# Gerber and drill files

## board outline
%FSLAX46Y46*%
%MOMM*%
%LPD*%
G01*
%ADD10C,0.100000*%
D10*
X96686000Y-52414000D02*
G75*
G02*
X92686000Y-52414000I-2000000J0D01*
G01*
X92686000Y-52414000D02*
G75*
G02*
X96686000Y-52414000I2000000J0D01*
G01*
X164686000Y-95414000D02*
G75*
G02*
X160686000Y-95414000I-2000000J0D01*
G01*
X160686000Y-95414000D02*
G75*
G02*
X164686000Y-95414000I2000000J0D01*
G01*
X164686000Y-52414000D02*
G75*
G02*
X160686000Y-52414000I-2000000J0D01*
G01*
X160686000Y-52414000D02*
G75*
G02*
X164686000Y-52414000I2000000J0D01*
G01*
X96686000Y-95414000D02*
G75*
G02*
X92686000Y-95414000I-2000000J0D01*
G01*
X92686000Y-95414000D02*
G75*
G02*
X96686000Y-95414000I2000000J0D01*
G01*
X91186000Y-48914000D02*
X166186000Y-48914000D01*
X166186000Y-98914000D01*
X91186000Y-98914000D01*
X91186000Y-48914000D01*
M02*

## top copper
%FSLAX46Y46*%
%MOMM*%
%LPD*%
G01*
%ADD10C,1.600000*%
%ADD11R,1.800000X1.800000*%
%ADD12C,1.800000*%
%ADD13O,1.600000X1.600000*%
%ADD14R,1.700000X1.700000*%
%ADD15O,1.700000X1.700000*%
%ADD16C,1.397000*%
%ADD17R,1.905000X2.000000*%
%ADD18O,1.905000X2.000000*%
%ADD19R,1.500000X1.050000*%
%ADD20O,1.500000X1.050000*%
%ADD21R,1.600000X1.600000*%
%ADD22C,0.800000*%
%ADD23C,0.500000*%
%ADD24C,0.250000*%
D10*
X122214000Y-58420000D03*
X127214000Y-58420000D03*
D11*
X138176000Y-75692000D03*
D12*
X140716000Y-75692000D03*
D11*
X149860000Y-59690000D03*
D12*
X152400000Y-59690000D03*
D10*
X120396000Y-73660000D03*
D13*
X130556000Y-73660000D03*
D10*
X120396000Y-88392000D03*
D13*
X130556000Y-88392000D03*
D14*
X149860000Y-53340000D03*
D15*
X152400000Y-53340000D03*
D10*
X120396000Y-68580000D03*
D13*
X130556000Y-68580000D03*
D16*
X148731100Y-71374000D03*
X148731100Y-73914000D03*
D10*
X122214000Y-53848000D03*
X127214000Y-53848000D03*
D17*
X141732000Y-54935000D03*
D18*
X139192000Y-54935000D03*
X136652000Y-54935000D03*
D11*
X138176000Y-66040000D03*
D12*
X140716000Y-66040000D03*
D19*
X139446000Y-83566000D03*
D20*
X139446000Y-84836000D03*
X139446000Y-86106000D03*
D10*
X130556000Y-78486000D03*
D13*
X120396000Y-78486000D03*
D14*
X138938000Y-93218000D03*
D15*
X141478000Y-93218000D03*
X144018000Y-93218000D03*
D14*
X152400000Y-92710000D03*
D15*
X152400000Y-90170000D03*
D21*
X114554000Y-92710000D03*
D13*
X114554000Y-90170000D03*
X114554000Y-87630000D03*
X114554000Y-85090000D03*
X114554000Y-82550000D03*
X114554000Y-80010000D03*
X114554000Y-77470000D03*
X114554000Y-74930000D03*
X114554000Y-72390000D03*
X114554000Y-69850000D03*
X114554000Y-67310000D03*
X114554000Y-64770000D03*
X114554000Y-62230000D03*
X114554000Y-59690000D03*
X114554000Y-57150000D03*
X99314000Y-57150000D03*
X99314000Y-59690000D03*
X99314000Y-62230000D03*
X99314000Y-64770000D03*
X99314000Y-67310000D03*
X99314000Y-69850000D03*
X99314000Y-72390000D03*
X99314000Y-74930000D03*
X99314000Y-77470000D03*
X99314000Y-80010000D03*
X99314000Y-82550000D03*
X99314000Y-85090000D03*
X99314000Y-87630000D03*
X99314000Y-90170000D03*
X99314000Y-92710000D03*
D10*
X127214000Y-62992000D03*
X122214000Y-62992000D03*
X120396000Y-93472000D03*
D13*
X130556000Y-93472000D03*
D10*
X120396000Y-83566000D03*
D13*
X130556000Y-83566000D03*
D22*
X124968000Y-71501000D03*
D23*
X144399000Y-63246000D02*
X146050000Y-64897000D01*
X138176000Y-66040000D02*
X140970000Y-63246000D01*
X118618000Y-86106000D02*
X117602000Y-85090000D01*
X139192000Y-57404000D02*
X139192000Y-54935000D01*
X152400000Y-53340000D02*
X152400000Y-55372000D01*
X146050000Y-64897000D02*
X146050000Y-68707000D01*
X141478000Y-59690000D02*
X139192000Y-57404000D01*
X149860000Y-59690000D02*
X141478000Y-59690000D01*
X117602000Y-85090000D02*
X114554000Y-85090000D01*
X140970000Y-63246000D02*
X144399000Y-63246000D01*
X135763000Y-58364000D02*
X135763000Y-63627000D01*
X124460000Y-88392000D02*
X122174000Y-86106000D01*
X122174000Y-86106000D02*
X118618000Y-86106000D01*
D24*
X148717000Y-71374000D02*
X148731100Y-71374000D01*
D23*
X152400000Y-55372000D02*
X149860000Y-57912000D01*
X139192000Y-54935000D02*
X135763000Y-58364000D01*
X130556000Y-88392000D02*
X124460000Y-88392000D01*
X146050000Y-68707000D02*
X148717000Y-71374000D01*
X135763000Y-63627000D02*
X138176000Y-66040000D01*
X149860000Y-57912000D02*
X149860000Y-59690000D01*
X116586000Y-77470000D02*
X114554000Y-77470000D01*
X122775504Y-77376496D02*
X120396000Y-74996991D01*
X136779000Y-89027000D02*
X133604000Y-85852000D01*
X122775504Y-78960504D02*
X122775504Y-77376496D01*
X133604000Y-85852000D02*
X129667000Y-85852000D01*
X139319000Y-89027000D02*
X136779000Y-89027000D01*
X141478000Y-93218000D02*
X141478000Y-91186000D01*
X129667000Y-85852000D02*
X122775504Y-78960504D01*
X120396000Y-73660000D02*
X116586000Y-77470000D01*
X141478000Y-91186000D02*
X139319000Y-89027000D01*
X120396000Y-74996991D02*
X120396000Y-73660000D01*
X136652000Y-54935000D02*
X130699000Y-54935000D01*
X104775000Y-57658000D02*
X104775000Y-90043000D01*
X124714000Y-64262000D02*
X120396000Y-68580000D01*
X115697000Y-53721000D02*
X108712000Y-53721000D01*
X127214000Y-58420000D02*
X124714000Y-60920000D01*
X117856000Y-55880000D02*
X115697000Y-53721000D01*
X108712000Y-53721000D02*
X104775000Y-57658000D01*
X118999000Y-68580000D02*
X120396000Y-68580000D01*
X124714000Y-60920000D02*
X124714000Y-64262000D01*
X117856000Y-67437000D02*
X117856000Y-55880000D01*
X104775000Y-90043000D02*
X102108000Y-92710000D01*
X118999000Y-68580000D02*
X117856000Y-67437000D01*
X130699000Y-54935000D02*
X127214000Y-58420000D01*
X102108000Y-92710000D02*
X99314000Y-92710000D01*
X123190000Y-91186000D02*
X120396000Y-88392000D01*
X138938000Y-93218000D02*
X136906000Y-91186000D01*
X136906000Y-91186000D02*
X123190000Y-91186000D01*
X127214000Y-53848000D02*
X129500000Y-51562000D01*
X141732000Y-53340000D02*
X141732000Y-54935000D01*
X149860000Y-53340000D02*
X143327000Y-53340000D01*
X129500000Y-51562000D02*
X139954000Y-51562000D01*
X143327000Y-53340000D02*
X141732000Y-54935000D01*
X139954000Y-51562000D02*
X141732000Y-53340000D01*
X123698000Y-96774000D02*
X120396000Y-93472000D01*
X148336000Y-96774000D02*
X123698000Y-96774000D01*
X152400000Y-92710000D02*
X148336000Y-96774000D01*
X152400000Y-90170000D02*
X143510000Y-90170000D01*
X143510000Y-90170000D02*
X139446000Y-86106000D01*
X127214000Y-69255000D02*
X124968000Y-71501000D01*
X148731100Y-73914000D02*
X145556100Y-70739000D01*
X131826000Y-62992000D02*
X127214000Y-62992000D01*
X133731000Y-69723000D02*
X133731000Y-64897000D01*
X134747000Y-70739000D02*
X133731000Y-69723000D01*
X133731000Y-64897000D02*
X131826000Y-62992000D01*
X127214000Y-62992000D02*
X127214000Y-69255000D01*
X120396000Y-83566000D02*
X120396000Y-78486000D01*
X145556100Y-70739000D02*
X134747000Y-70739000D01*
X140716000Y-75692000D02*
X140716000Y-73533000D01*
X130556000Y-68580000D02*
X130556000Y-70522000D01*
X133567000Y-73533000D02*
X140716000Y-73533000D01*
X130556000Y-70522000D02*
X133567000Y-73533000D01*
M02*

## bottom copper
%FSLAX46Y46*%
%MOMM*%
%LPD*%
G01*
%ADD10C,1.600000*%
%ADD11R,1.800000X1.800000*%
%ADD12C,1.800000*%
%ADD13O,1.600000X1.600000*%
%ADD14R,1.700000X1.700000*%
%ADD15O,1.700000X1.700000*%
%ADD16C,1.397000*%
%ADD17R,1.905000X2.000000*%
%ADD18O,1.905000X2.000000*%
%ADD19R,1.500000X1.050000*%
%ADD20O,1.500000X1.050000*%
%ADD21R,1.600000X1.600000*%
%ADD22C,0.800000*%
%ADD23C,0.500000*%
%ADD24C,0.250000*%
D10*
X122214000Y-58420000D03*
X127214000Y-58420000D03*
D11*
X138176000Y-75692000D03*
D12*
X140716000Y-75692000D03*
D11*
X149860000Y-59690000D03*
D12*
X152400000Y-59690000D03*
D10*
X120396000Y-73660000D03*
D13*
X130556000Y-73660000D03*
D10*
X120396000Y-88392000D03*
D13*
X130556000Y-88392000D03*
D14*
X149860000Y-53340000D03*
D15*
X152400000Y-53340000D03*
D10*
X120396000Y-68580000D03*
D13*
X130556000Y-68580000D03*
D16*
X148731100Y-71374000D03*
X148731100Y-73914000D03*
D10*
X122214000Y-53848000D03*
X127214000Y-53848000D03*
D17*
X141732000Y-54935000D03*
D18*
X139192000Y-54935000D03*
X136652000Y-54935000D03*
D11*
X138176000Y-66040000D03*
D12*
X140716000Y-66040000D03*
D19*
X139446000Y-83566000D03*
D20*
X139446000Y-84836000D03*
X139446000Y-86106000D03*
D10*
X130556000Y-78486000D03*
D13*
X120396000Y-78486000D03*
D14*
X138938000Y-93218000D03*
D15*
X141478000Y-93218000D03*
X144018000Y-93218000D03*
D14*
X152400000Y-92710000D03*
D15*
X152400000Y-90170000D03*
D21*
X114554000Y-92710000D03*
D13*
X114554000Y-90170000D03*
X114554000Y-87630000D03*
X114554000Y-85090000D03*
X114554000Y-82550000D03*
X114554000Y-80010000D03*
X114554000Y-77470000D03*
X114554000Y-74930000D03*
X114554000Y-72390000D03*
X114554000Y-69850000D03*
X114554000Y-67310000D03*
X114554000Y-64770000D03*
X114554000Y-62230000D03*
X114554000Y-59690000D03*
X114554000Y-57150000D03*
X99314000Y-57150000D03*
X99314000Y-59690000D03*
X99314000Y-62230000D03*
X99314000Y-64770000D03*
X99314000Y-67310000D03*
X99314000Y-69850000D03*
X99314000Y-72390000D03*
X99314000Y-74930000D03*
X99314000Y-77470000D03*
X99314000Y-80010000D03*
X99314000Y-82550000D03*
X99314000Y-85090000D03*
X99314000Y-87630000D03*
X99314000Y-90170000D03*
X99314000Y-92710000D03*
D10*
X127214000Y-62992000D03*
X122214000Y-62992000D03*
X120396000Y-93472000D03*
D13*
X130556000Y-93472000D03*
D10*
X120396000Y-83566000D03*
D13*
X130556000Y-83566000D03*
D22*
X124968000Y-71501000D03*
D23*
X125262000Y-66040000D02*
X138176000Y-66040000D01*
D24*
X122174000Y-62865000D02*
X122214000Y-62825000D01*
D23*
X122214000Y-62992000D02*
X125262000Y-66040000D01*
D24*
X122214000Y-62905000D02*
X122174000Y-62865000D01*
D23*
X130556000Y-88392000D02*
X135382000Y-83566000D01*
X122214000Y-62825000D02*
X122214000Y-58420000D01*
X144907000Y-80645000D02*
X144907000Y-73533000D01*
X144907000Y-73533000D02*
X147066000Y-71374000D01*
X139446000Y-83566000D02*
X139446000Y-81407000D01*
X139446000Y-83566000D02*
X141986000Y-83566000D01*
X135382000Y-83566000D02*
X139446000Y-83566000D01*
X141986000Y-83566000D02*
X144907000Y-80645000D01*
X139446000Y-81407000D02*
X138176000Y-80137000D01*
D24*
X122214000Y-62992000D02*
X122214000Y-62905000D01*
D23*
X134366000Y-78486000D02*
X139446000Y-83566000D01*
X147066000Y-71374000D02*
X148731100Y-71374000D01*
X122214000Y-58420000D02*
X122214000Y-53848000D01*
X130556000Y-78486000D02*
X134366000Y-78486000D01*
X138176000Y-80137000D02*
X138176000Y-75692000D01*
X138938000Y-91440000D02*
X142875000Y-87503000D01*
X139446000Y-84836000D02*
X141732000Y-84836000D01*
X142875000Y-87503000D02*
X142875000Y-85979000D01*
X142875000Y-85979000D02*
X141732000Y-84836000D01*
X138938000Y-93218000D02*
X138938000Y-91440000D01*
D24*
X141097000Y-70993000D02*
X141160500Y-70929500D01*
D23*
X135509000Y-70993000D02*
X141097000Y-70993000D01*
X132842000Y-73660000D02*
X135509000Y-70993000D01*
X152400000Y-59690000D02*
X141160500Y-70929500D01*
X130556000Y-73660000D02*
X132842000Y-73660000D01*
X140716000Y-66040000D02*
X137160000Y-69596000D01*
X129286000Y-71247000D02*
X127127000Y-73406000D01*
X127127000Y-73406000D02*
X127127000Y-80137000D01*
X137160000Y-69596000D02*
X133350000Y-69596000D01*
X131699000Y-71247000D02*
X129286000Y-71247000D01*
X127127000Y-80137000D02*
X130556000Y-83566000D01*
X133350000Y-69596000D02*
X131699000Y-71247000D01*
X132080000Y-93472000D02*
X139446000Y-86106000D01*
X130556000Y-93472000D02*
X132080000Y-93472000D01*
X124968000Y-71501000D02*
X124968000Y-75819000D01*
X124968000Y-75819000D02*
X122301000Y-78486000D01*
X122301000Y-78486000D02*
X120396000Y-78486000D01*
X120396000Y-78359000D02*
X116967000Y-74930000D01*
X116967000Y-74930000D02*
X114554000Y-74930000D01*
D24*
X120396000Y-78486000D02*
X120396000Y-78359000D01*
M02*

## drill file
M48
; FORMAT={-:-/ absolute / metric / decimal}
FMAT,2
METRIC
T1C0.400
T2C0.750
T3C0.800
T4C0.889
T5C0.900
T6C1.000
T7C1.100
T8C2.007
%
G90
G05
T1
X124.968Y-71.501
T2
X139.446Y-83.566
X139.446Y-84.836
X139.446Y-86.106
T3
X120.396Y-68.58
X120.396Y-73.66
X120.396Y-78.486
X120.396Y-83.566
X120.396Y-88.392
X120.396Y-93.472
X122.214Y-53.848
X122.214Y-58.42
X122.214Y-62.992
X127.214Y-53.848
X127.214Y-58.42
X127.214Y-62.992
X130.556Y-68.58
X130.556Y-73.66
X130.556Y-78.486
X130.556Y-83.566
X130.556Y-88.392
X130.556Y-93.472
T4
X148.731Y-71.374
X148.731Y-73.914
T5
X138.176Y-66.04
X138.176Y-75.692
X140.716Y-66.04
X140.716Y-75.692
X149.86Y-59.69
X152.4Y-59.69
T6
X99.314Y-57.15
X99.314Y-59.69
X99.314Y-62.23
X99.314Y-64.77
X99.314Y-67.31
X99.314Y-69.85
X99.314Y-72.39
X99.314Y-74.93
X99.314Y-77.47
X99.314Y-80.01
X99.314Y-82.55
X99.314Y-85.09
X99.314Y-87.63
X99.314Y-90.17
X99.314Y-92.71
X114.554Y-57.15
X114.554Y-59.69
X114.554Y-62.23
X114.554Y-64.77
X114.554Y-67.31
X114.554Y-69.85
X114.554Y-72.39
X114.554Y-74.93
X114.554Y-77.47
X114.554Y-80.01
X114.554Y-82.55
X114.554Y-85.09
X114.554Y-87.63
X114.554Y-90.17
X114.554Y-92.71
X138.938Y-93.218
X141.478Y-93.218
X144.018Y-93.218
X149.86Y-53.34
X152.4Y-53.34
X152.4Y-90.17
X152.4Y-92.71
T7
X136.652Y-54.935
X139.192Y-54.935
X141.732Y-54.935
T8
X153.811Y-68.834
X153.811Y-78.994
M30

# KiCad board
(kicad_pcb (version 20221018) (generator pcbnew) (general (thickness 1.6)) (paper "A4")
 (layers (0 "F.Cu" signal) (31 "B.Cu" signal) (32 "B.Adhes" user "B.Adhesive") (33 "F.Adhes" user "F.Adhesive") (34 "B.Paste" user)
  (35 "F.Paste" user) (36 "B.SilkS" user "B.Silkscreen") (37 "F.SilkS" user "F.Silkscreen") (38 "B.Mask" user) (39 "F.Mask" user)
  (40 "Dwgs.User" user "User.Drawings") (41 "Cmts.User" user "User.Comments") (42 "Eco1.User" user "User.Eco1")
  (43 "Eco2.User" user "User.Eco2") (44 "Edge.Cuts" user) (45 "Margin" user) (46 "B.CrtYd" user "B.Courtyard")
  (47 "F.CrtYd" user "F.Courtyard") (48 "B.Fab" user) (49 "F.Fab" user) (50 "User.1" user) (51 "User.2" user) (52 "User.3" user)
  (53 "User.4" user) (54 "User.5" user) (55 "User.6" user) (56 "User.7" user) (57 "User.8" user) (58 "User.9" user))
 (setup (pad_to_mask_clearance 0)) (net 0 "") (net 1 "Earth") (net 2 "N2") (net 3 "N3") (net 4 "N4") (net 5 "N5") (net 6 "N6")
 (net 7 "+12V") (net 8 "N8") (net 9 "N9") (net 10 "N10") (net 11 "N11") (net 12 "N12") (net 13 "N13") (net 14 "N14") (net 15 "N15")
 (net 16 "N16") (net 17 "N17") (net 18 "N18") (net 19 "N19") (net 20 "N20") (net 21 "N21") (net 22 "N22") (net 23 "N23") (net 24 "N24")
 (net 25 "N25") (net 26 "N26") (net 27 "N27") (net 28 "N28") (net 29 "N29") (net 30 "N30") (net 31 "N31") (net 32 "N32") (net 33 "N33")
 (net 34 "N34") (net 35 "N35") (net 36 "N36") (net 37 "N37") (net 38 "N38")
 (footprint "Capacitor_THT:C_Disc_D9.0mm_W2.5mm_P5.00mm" (layer "F.Cu") (at 122.214 58.42)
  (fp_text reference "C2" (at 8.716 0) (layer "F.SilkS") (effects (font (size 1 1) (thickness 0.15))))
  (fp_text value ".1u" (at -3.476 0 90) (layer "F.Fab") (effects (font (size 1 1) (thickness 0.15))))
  (pad "1" thru_hole circle (at 0 0) (size 1.6 1.6) (drill 0.8) (layers "*.Cu" "*.Mask") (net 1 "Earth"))
  (pad "2" thru_hole circle (at 5 0) (size 1.6 1.6) (drill 0.8) (layers "*.Cu" "*.Mask") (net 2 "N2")))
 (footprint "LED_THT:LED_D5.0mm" (layer "F.Cu") (at 138.176 75.692)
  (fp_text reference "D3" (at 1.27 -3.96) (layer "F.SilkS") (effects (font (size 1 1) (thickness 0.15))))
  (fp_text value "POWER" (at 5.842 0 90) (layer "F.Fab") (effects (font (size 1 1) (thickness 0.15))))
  (pad "1" thru_hole rect (at 0 0) (size 1.8 1.8) (drill 0.9) (layers "*.Cu" "*.Mask") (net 1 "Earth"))
  (pad "2" thru_hole circle (at 2.54 0) (size 1.8 1.8) (drill 0.9) (layers "*.Cu" "*.Mask") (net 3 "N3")))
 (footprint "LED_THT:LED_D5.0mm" (layer "F.Cu") (at 149.86 59.69)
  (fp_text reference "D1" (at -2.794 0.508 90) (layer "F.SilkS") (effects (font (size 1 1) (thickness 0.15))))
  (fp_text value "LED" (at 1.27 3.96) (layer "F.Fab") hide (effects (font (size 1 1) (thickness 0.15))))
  (pad "1" thru_hole rect (at 0 0) (size 1.8 1.8) (drill 0.9) (layers "*.Cu" "*.Mask") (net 1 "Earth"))
  (pad "2" thru_hole circle (at 2.54 0) (size 1.8 1.8) (drill 0.9) (layers "*.Cu" "*.Mask") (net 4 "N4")))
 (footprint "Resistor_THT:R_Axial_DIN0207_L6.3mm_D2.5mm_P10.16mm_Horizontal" (layer "F.Cu") (at 120.396 73.66)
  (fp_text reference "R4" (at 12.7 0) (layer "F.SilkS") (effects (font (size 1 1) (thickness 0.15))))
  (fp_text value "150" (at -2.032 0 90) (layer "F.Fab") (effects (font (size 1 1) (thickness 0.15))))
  (pad "1" thru_hole circle (at 0 0) (size 1.6 1.6) (drill 0.8) (layers "*.Cu" "*.Mask") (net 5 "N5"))
  (pad "2" thru_hole oval (at 10.16 0) (size 1.6 1.6) (drill 0.8) (layers "*.Cu" "*.Mask") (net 4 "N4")))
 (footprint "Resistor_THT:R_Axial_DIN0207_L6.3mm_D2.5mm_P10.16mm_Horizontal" (layer "F.Cu") (at 120.396 88.392)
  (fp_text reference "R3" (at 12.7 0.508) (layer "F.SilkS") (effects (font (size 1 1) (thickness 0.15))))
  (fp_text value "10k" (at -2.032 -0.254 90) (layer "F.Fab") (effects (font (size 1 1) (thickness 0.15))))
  (pad "1" thru_hole circle (at 0 0) (size 1.6 1.6) (drill 0.8) (layers "*.Cu" "*.Mask") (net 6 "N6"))
  (pad "2" thru_hole oval (at 10.16 0) (size 1.6 1.6) (drill 0.8) (layers "*.Cu" "*.Mask") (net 1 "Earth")))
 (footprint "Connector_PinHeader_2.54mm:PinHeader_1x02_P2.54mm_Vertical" (layer "F.Cu") (at 149.86 53.34 90)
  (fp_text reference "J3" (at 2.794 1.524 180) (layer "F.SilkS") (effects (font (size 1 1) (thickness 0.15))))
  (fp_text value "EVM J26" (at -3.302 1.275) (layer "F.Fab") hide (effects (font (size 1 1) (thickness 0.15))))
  (pad "1" thru_hole rect (at 0 0 90) (size 1.7 1.7) (drill 1) (layers "*.Cu" "*.Mask") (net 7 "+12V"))
  (pad "2" thru_hole oval (at 0 2.54 90) (size 1.7 1.7) (drill 1) (layers "*.Cu" "*.Mask") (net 1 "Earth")))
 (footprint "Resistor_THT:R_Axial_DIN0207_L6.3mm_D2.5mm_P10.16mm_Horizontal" (layer "F.Cu") (at 120.396 68.58)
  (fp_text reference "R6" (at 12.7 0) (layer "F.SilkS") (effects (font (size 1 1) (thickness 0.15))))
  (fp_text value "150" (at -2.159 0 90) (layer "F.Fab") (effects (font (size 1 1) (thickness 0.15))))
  (pad "1" thru_hole circle (at 0 0) (size 1.6 1.6) (drill 0.8) (layers "*.Cu" "*.Mask") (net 2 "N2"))
  (pad "2" thru_hole oval (at 10.16 0) (size 1.6 1.6) (drill 0.8) (layers "*.Cu" "*.Mask") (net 3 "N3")))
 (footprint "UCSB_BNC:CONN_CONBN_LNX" (layer "F.Cu") (at 156.186 73.914 -90)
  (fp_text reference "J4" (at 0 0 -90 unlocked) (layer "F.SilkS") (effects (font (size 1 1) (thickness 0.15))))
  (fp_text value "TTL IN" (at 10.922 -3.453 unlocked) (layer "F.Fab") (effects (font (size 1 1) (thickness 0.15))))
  (pad "" np_thru_hole circle (at -5.08 2.3749 270) (size 2.0066 2.0066) (drill 2.0066) (layers "*.Cu" "*.Mask"))
  (pad "" np_thru_hole circle (at 5.08 2.3749 270) (size 2.0066 2.0066) (drill 2.0066) (layers "*.Cu" "*.Mask"))
  (pad "1" thru_hole circle (at -2.54 7.4549 270) (size 1.397 1.397) (drill 0.889) (layers "*.Cu" "*.Mask") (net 1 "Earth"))
  (pad "2" thru_hole circle (at 0 7.4549 270) (size 1.397 1.397) (drill 0.889) (layers "*.Cu" "*.Mask") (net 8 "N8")))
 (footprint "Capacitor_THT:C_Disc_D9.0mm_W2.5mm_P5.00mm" (layer "F.Cu") (at 122.214 53.848)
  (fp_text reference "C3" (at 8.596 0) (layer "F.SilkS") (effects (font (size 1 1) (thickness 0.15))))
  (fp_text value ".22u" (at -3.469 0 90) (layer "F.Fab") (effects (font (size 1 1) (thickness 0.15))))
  (pad "1" thru_hole circle (at 0 0) (size 1.6 1.6) (drill 0.8) (layers "*.Cu" "*.Mask") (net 1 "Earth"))
  (pad "2" thru_hole circle (at 5 0) (size 1.6 1.6) (drill 0.8) (layers "*.Cu" "*.Mask") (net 7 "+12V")))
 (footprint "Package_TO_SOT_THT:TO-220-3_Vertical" (layer "F.Cu") (at 141.732 54.935 180)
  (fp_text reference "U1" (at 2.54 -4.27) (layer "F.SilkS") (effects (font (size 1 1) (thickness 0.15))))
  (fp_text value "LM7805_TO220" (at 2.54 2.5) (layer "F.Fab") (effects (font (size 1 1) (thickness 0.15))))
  (pad "1" thru_hole rect (at 0 0 180) (size 1.905 2) (drill 1.1) (layers "*.Cu" "*.Mask") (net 7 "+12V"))
  (pad "2" thru_hole oval (at 2.54 0 180) (size 1.905 2) (drill 1.1) (layers "*.Cu" "*.Mask") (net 1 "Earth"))
  (pad "3" thru_hole oval (at 5.08 0 180) (size 1.905 2) (drill 1.1) (layers "*.Cu" "*.Mask") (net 2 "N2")))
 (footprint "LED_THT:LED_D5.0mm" (layer "F.Cu") (at 138.176 66.04)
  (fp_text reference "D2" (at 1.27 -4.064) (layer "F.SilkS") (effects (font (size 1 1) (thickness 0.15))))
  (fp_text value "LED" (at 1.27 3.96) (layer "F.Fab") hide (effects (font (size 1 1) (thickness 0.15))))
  (pad "1" thru_hole rect (at 0 0) (size 1.8 1.8) (drill 0.9) (layers "*.Cu" "*.Mask") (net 1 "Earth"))
  (pad "2" thru_hole circle (at 2.54 0) (size 1.8 1.8) (drill 0.9) (layers "*.Cu" "*.Mask") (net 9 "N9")))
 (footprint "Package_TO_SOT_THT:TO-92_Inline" (layer "F.Cu") (at 139.446 83.566 -90)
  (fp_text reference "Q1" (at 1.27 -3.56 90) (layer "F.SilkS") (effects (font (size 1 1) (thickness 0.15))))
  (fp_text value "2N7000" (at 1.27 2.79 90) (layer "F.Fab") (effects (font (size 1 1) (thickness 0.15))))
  (pad "1" thru_hole rect (at 0 0 270) (size 1.05 1.5) (drill 0.75) (layers "*.Cu" "*.Mask") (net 1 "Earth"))
  (pad "2" thru_hole oval (at 1.27 0 270) (size 1.05 1.5) (drill 0.75) (layers "*.Cu" "*.Mask") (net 6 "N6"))
  (pad "3" thru_hole oval (at 2.54 0 270) (size 1.05 1.5) (drill 0.75) (layers "*.Cu" "*.Mask") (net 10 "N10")))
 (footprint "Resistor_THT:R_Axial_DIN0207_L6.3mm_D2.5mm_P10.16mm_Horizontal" (layer "F.Cu") (at 130.556 78.486 180)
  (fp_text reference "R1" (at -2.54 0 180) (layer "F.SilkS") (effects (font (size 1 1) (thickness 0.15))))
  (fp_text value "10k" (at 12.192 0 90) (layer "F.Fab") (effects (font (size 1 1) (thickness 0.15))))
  (pad "1" thru_hole circle (at 0 0 180) (size 1.6 1.6) (drill 0.8) (layers "*.Cu" "*.Mask") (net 1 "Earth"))
  (pad "2" thru_hole oval (at 10.16 0 180) (size 1.6 1.6) (drill 0.8) (layers "*.Cu" "*.Mask") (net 8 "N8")))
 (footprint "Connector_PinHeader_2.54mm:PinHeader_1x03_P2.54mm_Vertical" (layer "F.Cu") (at 138.938 93.218 90)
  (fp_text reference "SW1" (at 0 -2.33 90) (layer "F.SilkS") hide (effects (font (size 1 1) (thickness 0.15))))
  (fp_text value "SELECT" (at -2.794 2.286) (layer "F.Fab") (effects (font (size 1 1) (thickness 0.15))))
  (pad "1" thru_hole rect (at 0 0 90) (size 1.7 1.7) (drill 1) (layers "*.Cu" "*.Mask") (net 6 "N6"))
  (pad "2" thru_hole oval (at 0 2.54 90) (size 1.7 1.7) (drill 1) (layers "*.Cu" "*.Mask") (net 5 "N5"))
  (pad "3" thru_hole oval (at 0 5.08 90) (size 1.7 1.7) (drill 1) (layers "*.Cu" "*.Mask") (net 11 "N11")))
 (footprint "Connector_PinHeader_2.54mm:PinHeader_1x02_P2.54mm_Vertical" (layer "F.Cu") (at 152.4 92.71 180)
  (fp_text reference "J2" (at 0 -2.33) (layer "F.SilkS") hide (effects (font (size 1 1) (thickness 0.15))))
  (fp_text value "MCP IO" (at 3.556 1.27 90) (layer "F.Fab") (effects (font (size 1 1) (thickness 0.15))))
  (pad "1" thru_hole rect (at 0 0 180) (size 1.7 1.7) (drill 1) (layers "*.Cu" "*.Mask") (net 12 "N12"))
  (pad "2" thru_hole oval (at 0 2.54 180) (size 1.7 1.7) (drill 1) (layers "*.Cu" "*.Mask") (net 10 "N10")))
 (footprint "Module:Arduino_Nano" (layer "F.Cu") (at 114.554 92.71 180)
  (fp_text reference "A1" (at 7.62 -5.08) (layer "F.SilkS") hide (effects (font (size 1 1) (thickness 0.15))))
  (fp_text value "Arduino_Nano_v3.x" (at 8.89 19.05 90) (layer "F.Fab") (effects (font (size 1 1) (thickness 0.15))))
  (pad "1" thru_hole rect (at 0 0 180) (size 1.6 1.6) (drill 1) (layers "*.Cu" "*.Mask") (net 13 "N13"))
  (pad "2" thru_hole oval (at 0 2.54 180) (size 1.6 1.6) (drill 1) (layers "*.Cu" "*.Mask") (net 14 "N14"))
  (pad "3" thru_hole oval (at 0 5.08 180) (size 1.6 1.6) (drill 1) (layers "*.Cu" "*.Mask") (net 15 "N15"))
  (pad "4" thru_hole oval (at 0 7.62 180) (size 1.6 1.6) (drill 1) (layers "*.Cu" "*.Mask") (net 1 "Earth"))
  (pad "5" thru_hole oval (at 0 10.16 180) (size 1.6 1.6) (drill 1) (layers "*.Cu" "*.Mask") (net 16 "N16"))
  (pad "6" thru_hole oval (at 0 12.7 180) (size 1.6 1.6) (drill 1) (layers "*.Cu" "*.Mask") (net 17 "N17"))
  (pad "7" thru_hole oval (at 0 15.24 180) (size 1.6 1.6) (drill 1) (layers "*.Cu" "*.Mask") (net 5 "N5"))
  (pad "8" thru_hole oval (at 0 17.78 180) (size 1.6 1.6) (drill 1) (layers "*.Cu" "*.Mask") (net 8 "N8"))
  (pad "9" thru_hole oval (at 0 20.32 180) (size 1.6 1.6) (drill 1) (layers "*.Cu" "*.Mask") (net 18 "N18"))
  (pad "10" thru_hole oval (at 0 22.86 180) (size 1.6 1.6) (drill 1) (layers "*.Cu" "*.Mask") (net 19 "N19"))
  (pad "11" thru_hole oval (at 0 25.4 180) (size 1.6 1.6) (drill 1) (layers "*.Cu" "*.Mask") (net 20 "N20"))
  (pad "12" thru_hole oval (at 0 27.94 180) (size 1.6 1.6) (drill 1) (layers "*.Cu" "*.Mask") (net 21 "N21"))
  (pad "13" thru_hole oval (at 0 30.48 180) (size 1.6 1.6) (drill 1) (layers "*.Cu" "*.Mask") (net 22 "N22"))
  (pad "14" thru_hole oval (at 0 33.02 180) (size 1.6 1.6) (drill 1) (layers "*.Cu" "*.Mask") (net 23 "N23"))
  (pad "15" thru_hole oval (at 0 35.56 180) (size 1.6 1.6) (drill 1) (layers "*.Cu" "*.Mask") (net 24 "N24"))
  (pad "16" thru_hole oval (at 15.24 35.56 180) (size 1.6 1.6) (drill 1) (layers "*.Cu" "*.Mask") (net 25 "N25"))
  (pad "17" thru_hole oval (at 15.24 33.02 180) (size 1.6 1.6) (drill 1) (layers "*.Cu" "*.Mask") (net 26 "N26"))
  (pad "18" thru_hole oval (at 15.24 30.48 180) (size 1.6 1.6) (drill 1) (layers "*.Cu" "*.Mask") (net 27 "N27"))
  (pad "19" thru_hole oval (at 15.24 27.94 180) (size 1.6 1.6) (drill 1) (layers "*.Cu" "*.Mask") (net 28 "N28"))
  (pad "20" thru_hole oval (at 15.24 25.4 180) (size 1.6 1.6) (drill 1) (layers "*.Cu" "*.Mask") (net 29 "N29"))
  (pad "21" thru_hole oval (at 15.24 22.86 180) (size 1.6 1.6) (drill 1) (layers "*.Cu" "*.Mask") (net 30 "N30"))
  (pad "22" thru_hole oval (at 15.24 20.32 180) (size 1.6 1.6) (drill 1) (layers "*.Cu" "*.Mask") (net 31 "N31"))
  (pad "23" thru_hole oval (at 15.24 17.78 180) (size 1.6 1.6) (drill 1) (layers "*.Cu" "*.Mask") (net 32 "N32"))
  (pad "24" thru_hole oval (at 15.24 15.24 180) (size 1.6 1.6) (drill 1) (layers "*.Cu" "*.Mask") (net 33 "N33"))
  (pad "25" thru_hole oval (at 15.24 12.7 180) (size 1.6 1.6) (drill 1) (layers "*.Cu" "*.Mask") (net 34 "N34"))
  (pad "26" thru_hole oval (at 15.24 10.16 180) (size 1.6 1.6) (drill 1) (layers "*.Cu" "*.Mask") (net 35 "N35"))
  (pad "27" thru_hole oval (at 15.24 7.62 180) (size 1.6 1.6) (drill 1) (layers "*.Cu" "*.Mask") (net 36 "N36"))
  (pad "28" thru_hole oval (at 15.24 5.08 180) (size 1.6 1.6) (drill 1) (layers "*.Cu" "*.Mask") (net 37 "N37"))
  (pad "29" thru_hole oval (at 15.24 2.54 180) (size 1.6 1.6) (drill 1) (layers "*.Cu" "*.Mask") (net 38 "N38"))
  (pad "30" thru_hole oval (at 15.24 0 180) (size 1.6 1.6) (drill 1) (layers "*.Cu" "*.Mask") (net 2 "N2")))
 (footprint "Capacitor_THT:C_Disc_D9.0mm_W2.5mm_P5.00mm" (layer "F.Cu") (at 127.214 62.992 180)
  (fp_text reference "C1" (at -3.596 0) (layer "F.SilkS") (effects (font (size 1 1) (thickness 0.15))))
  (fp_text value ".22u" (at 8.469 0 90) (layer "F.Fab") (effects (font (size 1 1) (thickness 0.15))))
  (pad "1" thru_hole circle (at 0 0 180) (size 1.6 1.6) (drill 0.8) (layers "*.Cu" "*.Mask") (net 8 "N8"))
  (pad "2" thru_hole circle (at 5 0 180) (size 1.6 1.6) (drill 0.8) (layers "*.Cu" "*.Mask") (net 1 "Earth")))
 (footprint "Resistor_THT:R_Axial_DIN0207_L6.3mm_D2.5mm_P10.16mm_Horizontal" (layer "F.Cu") (at 120.396 93.472)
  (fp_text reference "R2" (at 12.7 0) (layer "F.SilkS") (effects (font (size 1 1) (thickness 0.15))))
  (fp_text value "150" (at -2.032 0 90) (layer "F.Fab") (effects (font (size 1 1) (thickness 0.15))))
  (pad "1" thru_hole circle (at 0 0) (size 1.6 1.6) (drill 0.8) (layers "*.Cu" "*.Mask") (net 12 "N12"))
  (pad "2" thru_hole oval (at 10.16 0) (size 1.6 1.6) (drill 0.8) (layers "*.Cu" "*.Mask") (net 10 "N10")))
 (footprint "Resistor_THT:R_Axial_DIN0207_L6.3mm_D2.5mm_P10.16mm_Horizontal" (layer "F.Cu") (at 120.396 83.566)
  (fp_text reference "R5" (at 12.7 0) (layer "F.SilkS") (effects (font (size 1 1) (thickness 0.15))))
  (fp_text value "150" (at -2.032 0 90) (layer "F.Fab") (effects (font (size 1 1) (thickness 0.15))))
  (pad "1" thru_hole circle (at 0 0) (size 1.6 1.6) (drill 0.8) (layers "*.Cu" "*.Mask") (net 8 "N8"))
  (pad "2" thru_hole oval (at 10.16 0) (size 1.6 1.6) (drill 0.8) (layers "*.Cu" "*.Mask") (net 9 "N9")))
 (gr_circle (center 94.686 52.414) (end 96.686 52.414) (stroke (width 0.1) (type default)) (fill none) (layer "Edge.Cuts"))
 (gr_circle (center 162.686 95.414) (end 164.686 95.414) (stroke (width 0.1) (type default)) (fill none) (layer "Edge.Cuts"))
 (gr_circle (center 162.686 52.414) (end 164.686 52.414) (stroke (width 0.1) (type default)) (fill none) (layer "Edge.Cuts"))
 (gr_circle (center 94.686 95.414) (end 96.686 95.414) (stroke (width 0.1) (type default)) (fill none) (layer "Edge.Cuts"))
 (gr_rect (start 91.186 48.914) (end 166.186 98.914) (stroke (width 0.1) (type default)) (fill none) (layer "Edge.Cuts"))
 (segment (start 144.399 63.246) (end 146.05 64.897) (width 0.5) (layer "F.Cu") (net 1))
 (segment (start 138.176 66.04) (end 140.97 63.246) (width 0.5) (layer "F.Cu") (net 1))
 (segment (start 118.618 86.106) (end 117.602 85.09) (width 0.5) (layer "F.Cu") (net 1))
 (segment (start 139.192 57.404) (end 139.192 54.935) (width 0.5) (layer "F.Cu") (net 1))
 (segment (start 152.4 53.34) (end 152.4 55.372) (width 0.5) (layer "F.Cu") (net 1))
 (segment (start 146.05 64.897) (end 146.05 68.707) (width 0.5) (layer "F.Cu") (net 1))
 (segment (start 141.478 59.69) (end 139.192 57.404) (width 0.5) (layer "F.Cu") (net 1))
 (segment (start 149.86 59.69) (end 141.478 59.69) (width 0.5) (layer "F.Cu") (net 1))
 (segment (start 117.602 85.09) (end 114.554 85.09) (width 0.5) (layer "F.Cu") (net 1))
 (segment (start 140.97 63.246) (end 144.399 63.246) (width 0.5) (layer "F.Cu") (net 1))
 (segment (start 135.763 58.364) (end 135.763 63.627) (width 0.5) (layer "F.Cu") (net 1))
 (segment (start 124.46 88.392) (end 122.174 86.106) (width 0.5) (layer "F.Cu") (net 1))
 (segment (start 122.174 86.106) (end 118.618 86.106) (width 0.5) (layer "F.Cu") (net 1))
 (segment (start 148.717 71.374) (end 148.7311 71.374) (width 0.25) (layer "F.Cu") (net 1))
 (segment (start 152.4 55.372) (end 149.86 57.912) (width 0.5) (layer "F.Cu") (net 1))
 (segment (start 139.192 54.935) (end 135.763 58.364) (width 0.5) (layer "F.Cu") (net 1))
 (segment (start 130.556 88.392) (end 124.46 88.392) (width 0.5) (layer "F.Cu") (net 1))
 (segment (start 146.05 68.707) (end 148.717 71.374) (width 0.5) (layer "F.Cu") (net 1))
 (segment (start 135.763 63.627) (end 138.176 66.04) (width 0.5) (layer "F.Cu") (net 1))
 (segment (start 149.86 57.912) (end 149.86 59.69) (width 0.5) (layer "F.Cu") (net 1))
 (segment (start 125.262 66.04) (end 138.176 66.04) (width 0.5) (layer "B.Cu") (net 1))
 (segment (start 122.174 62.865) (end 122.214 62.825) (width 0.25) (layer "B.Cu") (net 1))
 (segment (start 122.214 62.992) (end 125.262 66.04) (width 0.5) (layer "B.Cu") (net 1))
 (segment (start 122.214 62.905) (end 122.174 62.865) (width 0.25) (layer "B.Cu") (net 1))
 (segment (start 130.556 88.392) (end 135.382 83.566) (width 0.5) (layer "B.Cu") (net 1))
 (segment (start 122.214 62.825) (end 122.214 58.42) (width 0.5) (layer "B.Cu") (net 1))
 (segment (start 144.907 80.645) (end 144.907 73.533) (width 0.5) (layer "B.Cu") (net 1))
 (segment (start 144.907 73.533) (end 147.066 71.374) (width 0.5) (layer "B.Cu") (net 1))
 (segment (start 139.446 83.566) (end 139.446 81.407) (width 0.5) (layer "B.Cu") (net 1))
 (segment (start 139.446 83.566) (end 141.986 83.566) (width 0.5) (layer "B.Cu") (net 1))
 (segment (start 135.382 83.566) (end 139.446 83.566) (width 0.5) (layer "B.Cu") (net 1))
 (segment (start 141.986 83.566) (end 144.907 80.645) (width 0.5) (layer "B.Cu") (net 1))
 (segment (start 139.446 81.407) (end 138.176 80.137) (width 0.5) (layer "B.Cu") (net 1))
 (segment (start 122.214 62.992) (end 122.214 62.905) (width 0.25) (layer "B.Cu") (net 1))
 (segment (start 134.366 78.486) (end 139.446 83.566) (width 0.5) (layer "B.Cu") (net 1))
 (segment (start 147.066 71.374) (end 148.7311 71.374) (width 0.5) (layer "B.Cu") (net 1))
 (segment (start 122.214 58.42) (end 122.214 53.848) (width 0.5) (layer "B.Cu") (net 1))
 (segment (start 130.556 78.486) (end 134.366 78.486) (width 0.5) (layer "B.Cu") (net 1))
 (segment (start 138.176 80.137) (end 138.176 75.692) (width 0.5) (layer "B.Cu") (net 1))
 (segment (start 116.586 77.47) (end 114.554 77.47) (width 0.5) (layer "F.Cu") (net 5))
 (segment (start 122.775504 77.376496) (end 120.396 74.996991) (width 0.5) (layer "F.Cu") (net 5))
 (segment (start 136.779 89.027) (end 133.604 85.852) (width 0.5) (layer "F.Cu") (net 5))
 (segment (start 122.775504 78.960504) (end 122.775504 77.376496) (width 0.5) (layer "F.Cu") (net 5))
 (segment (start 133.604 85.852) (end 129.667 85.852) (width 0.5) (layer "F.Cu") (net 5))
 (segment (start 139.319 89.027) (end 136.779 89.027) (width 0.5) (layer "F.Cu") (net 5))
 (segment (start 141.478 93.218) (end 141.478 91.186) (width 0.5) (layer "F.Cu") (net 5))
 (segment (start 129.667 85.852) (end 122.775504 78.960504) (width 0.5) (layer "F.Cu") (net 5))
 (segment (start 120.396 73.66) (end 116.586 77.47) (width 0.5) (layer "F.Cu") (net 5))
 (segment (start 141.478 91.186) (end 139.319 89.027) (width 0.5) (layer "F.Cu") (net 5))
 (segment (start 120.396 74.996991) (end 120.396 73.66) (width 0.5) (layer "F.Cu") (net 5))
 (segment (start 136.652 54.935) (end 130.699 54.935) (width 0.5) (layer "F.Cu") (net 2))
 (segment (start 104.775 57.658) (end 104.775 90.043) (width 0.5) (layer "F.Cu") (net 2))
 (segment (start 124.714 64.262) (end 120.396 68.58) (width 0.5) (layer "F.Cu") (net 2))
 (segment (start 115.697 53.721) (end 108.712 53.721) (width 0.5) (layer "F.Cu") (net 2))
 (segment (start 127.214 58.42) (end 124.714 60.92) (width 0.5) (layer "F.Cu") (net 2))
 (segment (start 117.856 55.88) (end 115.697 53.721) (width 0.5) (layer "F.Cu") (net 2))
 (segment (start 108.712 53.721) (end 104.775 57.658) (width 0.5) (layer "F.Cu") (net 2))
 (segment (start 118.999 68.58) (end 120.396 68.58) (width 0.5) (layer "F.Cu") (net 2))
 (segment (start 124.714 60.92) (end 124.714 64.262) (width 0.5) (layer "F.Cu") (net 2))
 (segment (start 117.856 67.437) (end 117.856 55.88) (width 0.5) (layer "F.Cu") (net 2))
 (segment (start 104.775 90.043) (end 102.108 92.71) (width 0.5) (layer "F.Cu") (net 2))
 (segment (start 118.999 68.58) (end 117.856 67.437) (width 0.5) (layer "F.Cu") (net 2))
 (segment (start 130.699 54.935) (end 127.214 58.42) (width 0.5) (layer "F.Cu") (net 2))
 (segment (start 102.108 92.71) (end 99.314 92.71) (width 0.5) (layer "F.Cu") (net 2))
 (segment (start 123.19 91.186) (end 120.396 88.392) (width 0.5) (layer "F.Cu") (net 6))
 (segment (start 138.938 93.218) (end 136.906 91.186) (width 0.5) (layer "F.Cu") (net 6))
 (segment (start 136.906 91.186) (end 123.19 91.186) (width 0.5) (layer "F.Cu") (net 6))
 (segment (start 138.938 91.44) (end 142.875 87.503) (width 0.5) (layer "B.Cu") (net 6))
 (segment (start 139.446 84.836) (end 141.732 84.836) (width 0.5) (layer "B.Cu") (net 6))
 (segment (start 142.875 87.503) (end 142.875 85.979) (width 0.5) (layer "B.Cu") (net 6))
 (segment (start 142.875 85.979) (end 141.732 84.836) (width 0.5) (layer "B.Cu") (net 6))
 (segment (start 138.938 93.218) (end 138.938 91.44) (width 0.5) (layer "B.Cu") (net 6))
 (segment (start 127.214 53.848) (end 129.5 51.562) (width 0.5) (layer "F.Cu") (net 7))
 (segment (start 141.732 53.34) (end 141.732 54.935) (width 0.5) (layer "F.Cu") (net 7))
 (segment (start 149.86 53.34) (end 143.327 53.34) (width 0.5) (layer "F.Cu") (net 7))
 (segment (start 129.5 51.562) (end 139.954 51.562) (width 0.5) (layer "F.Cu") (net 7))
 (segment (start 143.327 53.34) (end 141.732 54.935) (width 0.5) (layer "F.Cu") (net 7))
 (segment (start 139.954 51.562) (end 141.732 53.34) (width 0.5) (layer "F.Cu") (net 7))
 (segment (start 141.097 70.993) (end 141.1605 70.9295) (width 0.25) (layer "B.Cu") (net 4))
 (segment (start 135.509 70.993) (end 141.097 70.993) (width 0.5) (layer "B.Cu") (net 4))
 (segment (start 132.842 73.66) (end 135.509 70.993) (width 0.5) (layer "B.Cu") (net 4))
 (segment (start 152.4 59.69) (end 141.1605 70.9295) (width 0.5) (layer "B.Cu") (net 4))
 (segment (start 130.556 73.66) (end 132.842 73.66) (width 0.5) (layer "B.Cu") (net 4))
 (segment (start 140.716 66.04) (end 137.16 69.596) (width 0.5) (layer "B.Cu") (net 9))
 (segment (start 129.286 71.247) (end 127.127 73.406) (width 0.5) (layer "B.Cu") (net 9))
 (segment (start 127.127 73.406) (end 127.127 80.137) (width 0.5) (layer "B.Cu") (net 9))
 (segment (start 137.16 69.596) (end 133.35 69.596) (width 0.5) (layer "B.Cu") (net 9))
 (segment (start 131.699 71.247) (end 129.286 71.247) (width 0.5) (layer "B.Cu") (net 9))
 (segment (start 127.127 80.137) (end 130.556 83.566) (width 0.5) (layer "B.Cu") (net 9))
 (segment (start 133.35 69.596) (end 131.699 71.247) (width 0.5) (layer "B.Cu") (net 9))
 (segment (start 123.698 96.774) (end 120.396 93.472) (width 0.5) (layer "F.Cu") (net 12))
 (segment (start 148.336 96.774) (end 123.698 96.774) (width 0.5) (layer "F.Cu") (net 12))
 (segment (start 152.4 92.71) (end 148.336 96.774) (width 0.5) (layer "F.Cu") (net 12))
 (segment (start 152.4 90.17) (end 143.51 90.17) (width 0.5) (layer "F.Cu") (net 10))
 (segment (start 143.51 90.17) (end 139.446 86.106) (width 0.5) (layer "F.Cu") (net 10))
 (segment (start 132.08 93.472) (end 139.446 86.106) (width 0.5) (layer "B.Cu") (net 10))
 (segment (start 130.556 93.472) (end 132.08 93.472) (width 0.5) (layer "B.Cu") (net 10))
 (segment (start 127.214 69.255) (end 124.968 71.501) (width 0.5) (layer "F.Cu") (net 8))
 (segment (start 148.7311 73.914) (end 145.5561 70.739) (width 0.5) (layer "F.Cu") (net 8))
 (segment (start 131.826 62.992) (end 127.214 62.992) (width 0.5) (layer "F.Cu") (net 8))
 (segment (start 133.731 69.723) (end 133.731 64.897) (width 0.5) (layer "F.Cu") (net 8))
 (segment (start 134.747 70.739) (end 133.731 69.723) (width 0.5) (layer "F.Cu") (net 8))
 (segment (start 133.731 64.897) (end 131.826 62.992) (width 0.5) (layer "F.Cu") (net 8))
 (segment (start 127.214 62.992) (end 127.214 69.255) (width 0.5) (layer "F.Cu") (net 8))
 (segment (start 120.396 83.566) (end 120.396 78.486) (width 0.5) (layer "F.Cu") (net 8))
 (segment (start 145.5561 70.739) (end 134.747 70.739) (width 0.5) (layer "F.Cu") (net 8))
 (via (at 124.968 71.501) (size 0.8) (drill 0.4) (layers "F.Cu" "B.Cu") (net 8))
 (segment (start 124.968 71.501) (end 124.968 75.819) (width 0.5) (layer "B.Cu") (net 8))
 (segment (start 124.968 75.819) (end 122.301 78.486) (width 0.5) (layer "B.Cu") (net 8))
 (segment (start 122.301 78.486) (end 120.396 78.486) (width 0.5) (layer "B.Cu") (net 8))
 (segment (start 120.396 78.359) (end 116.967 74.93) (width 0.5) (layer "B.Cu") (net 8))
 (segment (start 116.967 74.93) (end 114.554 74.93) (width 0.5) (layer "B.Cu") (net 8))
 (segment (start 120.396 78.486) (end 120.396 78.359) (width 0.25) (layer "B.Cu") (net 8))
 (segment (start 140.716 75.692) (end 140.716 73.533) (width 0.5) (layer "F.Cu") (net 3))
 (segment (start 130.556 68.58) (end 130.556 70.522) (width 0.5) (layer "F.Cu") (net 3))
 (segment (start 133.567 73.533) (end 140.716 73.533) (width 0.5) (layer "F.Cu") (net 3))
 (segment (start 130.556 70.522) (end 133.567 73.533) (width 0.5) (layer "F.Cu") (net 3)))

